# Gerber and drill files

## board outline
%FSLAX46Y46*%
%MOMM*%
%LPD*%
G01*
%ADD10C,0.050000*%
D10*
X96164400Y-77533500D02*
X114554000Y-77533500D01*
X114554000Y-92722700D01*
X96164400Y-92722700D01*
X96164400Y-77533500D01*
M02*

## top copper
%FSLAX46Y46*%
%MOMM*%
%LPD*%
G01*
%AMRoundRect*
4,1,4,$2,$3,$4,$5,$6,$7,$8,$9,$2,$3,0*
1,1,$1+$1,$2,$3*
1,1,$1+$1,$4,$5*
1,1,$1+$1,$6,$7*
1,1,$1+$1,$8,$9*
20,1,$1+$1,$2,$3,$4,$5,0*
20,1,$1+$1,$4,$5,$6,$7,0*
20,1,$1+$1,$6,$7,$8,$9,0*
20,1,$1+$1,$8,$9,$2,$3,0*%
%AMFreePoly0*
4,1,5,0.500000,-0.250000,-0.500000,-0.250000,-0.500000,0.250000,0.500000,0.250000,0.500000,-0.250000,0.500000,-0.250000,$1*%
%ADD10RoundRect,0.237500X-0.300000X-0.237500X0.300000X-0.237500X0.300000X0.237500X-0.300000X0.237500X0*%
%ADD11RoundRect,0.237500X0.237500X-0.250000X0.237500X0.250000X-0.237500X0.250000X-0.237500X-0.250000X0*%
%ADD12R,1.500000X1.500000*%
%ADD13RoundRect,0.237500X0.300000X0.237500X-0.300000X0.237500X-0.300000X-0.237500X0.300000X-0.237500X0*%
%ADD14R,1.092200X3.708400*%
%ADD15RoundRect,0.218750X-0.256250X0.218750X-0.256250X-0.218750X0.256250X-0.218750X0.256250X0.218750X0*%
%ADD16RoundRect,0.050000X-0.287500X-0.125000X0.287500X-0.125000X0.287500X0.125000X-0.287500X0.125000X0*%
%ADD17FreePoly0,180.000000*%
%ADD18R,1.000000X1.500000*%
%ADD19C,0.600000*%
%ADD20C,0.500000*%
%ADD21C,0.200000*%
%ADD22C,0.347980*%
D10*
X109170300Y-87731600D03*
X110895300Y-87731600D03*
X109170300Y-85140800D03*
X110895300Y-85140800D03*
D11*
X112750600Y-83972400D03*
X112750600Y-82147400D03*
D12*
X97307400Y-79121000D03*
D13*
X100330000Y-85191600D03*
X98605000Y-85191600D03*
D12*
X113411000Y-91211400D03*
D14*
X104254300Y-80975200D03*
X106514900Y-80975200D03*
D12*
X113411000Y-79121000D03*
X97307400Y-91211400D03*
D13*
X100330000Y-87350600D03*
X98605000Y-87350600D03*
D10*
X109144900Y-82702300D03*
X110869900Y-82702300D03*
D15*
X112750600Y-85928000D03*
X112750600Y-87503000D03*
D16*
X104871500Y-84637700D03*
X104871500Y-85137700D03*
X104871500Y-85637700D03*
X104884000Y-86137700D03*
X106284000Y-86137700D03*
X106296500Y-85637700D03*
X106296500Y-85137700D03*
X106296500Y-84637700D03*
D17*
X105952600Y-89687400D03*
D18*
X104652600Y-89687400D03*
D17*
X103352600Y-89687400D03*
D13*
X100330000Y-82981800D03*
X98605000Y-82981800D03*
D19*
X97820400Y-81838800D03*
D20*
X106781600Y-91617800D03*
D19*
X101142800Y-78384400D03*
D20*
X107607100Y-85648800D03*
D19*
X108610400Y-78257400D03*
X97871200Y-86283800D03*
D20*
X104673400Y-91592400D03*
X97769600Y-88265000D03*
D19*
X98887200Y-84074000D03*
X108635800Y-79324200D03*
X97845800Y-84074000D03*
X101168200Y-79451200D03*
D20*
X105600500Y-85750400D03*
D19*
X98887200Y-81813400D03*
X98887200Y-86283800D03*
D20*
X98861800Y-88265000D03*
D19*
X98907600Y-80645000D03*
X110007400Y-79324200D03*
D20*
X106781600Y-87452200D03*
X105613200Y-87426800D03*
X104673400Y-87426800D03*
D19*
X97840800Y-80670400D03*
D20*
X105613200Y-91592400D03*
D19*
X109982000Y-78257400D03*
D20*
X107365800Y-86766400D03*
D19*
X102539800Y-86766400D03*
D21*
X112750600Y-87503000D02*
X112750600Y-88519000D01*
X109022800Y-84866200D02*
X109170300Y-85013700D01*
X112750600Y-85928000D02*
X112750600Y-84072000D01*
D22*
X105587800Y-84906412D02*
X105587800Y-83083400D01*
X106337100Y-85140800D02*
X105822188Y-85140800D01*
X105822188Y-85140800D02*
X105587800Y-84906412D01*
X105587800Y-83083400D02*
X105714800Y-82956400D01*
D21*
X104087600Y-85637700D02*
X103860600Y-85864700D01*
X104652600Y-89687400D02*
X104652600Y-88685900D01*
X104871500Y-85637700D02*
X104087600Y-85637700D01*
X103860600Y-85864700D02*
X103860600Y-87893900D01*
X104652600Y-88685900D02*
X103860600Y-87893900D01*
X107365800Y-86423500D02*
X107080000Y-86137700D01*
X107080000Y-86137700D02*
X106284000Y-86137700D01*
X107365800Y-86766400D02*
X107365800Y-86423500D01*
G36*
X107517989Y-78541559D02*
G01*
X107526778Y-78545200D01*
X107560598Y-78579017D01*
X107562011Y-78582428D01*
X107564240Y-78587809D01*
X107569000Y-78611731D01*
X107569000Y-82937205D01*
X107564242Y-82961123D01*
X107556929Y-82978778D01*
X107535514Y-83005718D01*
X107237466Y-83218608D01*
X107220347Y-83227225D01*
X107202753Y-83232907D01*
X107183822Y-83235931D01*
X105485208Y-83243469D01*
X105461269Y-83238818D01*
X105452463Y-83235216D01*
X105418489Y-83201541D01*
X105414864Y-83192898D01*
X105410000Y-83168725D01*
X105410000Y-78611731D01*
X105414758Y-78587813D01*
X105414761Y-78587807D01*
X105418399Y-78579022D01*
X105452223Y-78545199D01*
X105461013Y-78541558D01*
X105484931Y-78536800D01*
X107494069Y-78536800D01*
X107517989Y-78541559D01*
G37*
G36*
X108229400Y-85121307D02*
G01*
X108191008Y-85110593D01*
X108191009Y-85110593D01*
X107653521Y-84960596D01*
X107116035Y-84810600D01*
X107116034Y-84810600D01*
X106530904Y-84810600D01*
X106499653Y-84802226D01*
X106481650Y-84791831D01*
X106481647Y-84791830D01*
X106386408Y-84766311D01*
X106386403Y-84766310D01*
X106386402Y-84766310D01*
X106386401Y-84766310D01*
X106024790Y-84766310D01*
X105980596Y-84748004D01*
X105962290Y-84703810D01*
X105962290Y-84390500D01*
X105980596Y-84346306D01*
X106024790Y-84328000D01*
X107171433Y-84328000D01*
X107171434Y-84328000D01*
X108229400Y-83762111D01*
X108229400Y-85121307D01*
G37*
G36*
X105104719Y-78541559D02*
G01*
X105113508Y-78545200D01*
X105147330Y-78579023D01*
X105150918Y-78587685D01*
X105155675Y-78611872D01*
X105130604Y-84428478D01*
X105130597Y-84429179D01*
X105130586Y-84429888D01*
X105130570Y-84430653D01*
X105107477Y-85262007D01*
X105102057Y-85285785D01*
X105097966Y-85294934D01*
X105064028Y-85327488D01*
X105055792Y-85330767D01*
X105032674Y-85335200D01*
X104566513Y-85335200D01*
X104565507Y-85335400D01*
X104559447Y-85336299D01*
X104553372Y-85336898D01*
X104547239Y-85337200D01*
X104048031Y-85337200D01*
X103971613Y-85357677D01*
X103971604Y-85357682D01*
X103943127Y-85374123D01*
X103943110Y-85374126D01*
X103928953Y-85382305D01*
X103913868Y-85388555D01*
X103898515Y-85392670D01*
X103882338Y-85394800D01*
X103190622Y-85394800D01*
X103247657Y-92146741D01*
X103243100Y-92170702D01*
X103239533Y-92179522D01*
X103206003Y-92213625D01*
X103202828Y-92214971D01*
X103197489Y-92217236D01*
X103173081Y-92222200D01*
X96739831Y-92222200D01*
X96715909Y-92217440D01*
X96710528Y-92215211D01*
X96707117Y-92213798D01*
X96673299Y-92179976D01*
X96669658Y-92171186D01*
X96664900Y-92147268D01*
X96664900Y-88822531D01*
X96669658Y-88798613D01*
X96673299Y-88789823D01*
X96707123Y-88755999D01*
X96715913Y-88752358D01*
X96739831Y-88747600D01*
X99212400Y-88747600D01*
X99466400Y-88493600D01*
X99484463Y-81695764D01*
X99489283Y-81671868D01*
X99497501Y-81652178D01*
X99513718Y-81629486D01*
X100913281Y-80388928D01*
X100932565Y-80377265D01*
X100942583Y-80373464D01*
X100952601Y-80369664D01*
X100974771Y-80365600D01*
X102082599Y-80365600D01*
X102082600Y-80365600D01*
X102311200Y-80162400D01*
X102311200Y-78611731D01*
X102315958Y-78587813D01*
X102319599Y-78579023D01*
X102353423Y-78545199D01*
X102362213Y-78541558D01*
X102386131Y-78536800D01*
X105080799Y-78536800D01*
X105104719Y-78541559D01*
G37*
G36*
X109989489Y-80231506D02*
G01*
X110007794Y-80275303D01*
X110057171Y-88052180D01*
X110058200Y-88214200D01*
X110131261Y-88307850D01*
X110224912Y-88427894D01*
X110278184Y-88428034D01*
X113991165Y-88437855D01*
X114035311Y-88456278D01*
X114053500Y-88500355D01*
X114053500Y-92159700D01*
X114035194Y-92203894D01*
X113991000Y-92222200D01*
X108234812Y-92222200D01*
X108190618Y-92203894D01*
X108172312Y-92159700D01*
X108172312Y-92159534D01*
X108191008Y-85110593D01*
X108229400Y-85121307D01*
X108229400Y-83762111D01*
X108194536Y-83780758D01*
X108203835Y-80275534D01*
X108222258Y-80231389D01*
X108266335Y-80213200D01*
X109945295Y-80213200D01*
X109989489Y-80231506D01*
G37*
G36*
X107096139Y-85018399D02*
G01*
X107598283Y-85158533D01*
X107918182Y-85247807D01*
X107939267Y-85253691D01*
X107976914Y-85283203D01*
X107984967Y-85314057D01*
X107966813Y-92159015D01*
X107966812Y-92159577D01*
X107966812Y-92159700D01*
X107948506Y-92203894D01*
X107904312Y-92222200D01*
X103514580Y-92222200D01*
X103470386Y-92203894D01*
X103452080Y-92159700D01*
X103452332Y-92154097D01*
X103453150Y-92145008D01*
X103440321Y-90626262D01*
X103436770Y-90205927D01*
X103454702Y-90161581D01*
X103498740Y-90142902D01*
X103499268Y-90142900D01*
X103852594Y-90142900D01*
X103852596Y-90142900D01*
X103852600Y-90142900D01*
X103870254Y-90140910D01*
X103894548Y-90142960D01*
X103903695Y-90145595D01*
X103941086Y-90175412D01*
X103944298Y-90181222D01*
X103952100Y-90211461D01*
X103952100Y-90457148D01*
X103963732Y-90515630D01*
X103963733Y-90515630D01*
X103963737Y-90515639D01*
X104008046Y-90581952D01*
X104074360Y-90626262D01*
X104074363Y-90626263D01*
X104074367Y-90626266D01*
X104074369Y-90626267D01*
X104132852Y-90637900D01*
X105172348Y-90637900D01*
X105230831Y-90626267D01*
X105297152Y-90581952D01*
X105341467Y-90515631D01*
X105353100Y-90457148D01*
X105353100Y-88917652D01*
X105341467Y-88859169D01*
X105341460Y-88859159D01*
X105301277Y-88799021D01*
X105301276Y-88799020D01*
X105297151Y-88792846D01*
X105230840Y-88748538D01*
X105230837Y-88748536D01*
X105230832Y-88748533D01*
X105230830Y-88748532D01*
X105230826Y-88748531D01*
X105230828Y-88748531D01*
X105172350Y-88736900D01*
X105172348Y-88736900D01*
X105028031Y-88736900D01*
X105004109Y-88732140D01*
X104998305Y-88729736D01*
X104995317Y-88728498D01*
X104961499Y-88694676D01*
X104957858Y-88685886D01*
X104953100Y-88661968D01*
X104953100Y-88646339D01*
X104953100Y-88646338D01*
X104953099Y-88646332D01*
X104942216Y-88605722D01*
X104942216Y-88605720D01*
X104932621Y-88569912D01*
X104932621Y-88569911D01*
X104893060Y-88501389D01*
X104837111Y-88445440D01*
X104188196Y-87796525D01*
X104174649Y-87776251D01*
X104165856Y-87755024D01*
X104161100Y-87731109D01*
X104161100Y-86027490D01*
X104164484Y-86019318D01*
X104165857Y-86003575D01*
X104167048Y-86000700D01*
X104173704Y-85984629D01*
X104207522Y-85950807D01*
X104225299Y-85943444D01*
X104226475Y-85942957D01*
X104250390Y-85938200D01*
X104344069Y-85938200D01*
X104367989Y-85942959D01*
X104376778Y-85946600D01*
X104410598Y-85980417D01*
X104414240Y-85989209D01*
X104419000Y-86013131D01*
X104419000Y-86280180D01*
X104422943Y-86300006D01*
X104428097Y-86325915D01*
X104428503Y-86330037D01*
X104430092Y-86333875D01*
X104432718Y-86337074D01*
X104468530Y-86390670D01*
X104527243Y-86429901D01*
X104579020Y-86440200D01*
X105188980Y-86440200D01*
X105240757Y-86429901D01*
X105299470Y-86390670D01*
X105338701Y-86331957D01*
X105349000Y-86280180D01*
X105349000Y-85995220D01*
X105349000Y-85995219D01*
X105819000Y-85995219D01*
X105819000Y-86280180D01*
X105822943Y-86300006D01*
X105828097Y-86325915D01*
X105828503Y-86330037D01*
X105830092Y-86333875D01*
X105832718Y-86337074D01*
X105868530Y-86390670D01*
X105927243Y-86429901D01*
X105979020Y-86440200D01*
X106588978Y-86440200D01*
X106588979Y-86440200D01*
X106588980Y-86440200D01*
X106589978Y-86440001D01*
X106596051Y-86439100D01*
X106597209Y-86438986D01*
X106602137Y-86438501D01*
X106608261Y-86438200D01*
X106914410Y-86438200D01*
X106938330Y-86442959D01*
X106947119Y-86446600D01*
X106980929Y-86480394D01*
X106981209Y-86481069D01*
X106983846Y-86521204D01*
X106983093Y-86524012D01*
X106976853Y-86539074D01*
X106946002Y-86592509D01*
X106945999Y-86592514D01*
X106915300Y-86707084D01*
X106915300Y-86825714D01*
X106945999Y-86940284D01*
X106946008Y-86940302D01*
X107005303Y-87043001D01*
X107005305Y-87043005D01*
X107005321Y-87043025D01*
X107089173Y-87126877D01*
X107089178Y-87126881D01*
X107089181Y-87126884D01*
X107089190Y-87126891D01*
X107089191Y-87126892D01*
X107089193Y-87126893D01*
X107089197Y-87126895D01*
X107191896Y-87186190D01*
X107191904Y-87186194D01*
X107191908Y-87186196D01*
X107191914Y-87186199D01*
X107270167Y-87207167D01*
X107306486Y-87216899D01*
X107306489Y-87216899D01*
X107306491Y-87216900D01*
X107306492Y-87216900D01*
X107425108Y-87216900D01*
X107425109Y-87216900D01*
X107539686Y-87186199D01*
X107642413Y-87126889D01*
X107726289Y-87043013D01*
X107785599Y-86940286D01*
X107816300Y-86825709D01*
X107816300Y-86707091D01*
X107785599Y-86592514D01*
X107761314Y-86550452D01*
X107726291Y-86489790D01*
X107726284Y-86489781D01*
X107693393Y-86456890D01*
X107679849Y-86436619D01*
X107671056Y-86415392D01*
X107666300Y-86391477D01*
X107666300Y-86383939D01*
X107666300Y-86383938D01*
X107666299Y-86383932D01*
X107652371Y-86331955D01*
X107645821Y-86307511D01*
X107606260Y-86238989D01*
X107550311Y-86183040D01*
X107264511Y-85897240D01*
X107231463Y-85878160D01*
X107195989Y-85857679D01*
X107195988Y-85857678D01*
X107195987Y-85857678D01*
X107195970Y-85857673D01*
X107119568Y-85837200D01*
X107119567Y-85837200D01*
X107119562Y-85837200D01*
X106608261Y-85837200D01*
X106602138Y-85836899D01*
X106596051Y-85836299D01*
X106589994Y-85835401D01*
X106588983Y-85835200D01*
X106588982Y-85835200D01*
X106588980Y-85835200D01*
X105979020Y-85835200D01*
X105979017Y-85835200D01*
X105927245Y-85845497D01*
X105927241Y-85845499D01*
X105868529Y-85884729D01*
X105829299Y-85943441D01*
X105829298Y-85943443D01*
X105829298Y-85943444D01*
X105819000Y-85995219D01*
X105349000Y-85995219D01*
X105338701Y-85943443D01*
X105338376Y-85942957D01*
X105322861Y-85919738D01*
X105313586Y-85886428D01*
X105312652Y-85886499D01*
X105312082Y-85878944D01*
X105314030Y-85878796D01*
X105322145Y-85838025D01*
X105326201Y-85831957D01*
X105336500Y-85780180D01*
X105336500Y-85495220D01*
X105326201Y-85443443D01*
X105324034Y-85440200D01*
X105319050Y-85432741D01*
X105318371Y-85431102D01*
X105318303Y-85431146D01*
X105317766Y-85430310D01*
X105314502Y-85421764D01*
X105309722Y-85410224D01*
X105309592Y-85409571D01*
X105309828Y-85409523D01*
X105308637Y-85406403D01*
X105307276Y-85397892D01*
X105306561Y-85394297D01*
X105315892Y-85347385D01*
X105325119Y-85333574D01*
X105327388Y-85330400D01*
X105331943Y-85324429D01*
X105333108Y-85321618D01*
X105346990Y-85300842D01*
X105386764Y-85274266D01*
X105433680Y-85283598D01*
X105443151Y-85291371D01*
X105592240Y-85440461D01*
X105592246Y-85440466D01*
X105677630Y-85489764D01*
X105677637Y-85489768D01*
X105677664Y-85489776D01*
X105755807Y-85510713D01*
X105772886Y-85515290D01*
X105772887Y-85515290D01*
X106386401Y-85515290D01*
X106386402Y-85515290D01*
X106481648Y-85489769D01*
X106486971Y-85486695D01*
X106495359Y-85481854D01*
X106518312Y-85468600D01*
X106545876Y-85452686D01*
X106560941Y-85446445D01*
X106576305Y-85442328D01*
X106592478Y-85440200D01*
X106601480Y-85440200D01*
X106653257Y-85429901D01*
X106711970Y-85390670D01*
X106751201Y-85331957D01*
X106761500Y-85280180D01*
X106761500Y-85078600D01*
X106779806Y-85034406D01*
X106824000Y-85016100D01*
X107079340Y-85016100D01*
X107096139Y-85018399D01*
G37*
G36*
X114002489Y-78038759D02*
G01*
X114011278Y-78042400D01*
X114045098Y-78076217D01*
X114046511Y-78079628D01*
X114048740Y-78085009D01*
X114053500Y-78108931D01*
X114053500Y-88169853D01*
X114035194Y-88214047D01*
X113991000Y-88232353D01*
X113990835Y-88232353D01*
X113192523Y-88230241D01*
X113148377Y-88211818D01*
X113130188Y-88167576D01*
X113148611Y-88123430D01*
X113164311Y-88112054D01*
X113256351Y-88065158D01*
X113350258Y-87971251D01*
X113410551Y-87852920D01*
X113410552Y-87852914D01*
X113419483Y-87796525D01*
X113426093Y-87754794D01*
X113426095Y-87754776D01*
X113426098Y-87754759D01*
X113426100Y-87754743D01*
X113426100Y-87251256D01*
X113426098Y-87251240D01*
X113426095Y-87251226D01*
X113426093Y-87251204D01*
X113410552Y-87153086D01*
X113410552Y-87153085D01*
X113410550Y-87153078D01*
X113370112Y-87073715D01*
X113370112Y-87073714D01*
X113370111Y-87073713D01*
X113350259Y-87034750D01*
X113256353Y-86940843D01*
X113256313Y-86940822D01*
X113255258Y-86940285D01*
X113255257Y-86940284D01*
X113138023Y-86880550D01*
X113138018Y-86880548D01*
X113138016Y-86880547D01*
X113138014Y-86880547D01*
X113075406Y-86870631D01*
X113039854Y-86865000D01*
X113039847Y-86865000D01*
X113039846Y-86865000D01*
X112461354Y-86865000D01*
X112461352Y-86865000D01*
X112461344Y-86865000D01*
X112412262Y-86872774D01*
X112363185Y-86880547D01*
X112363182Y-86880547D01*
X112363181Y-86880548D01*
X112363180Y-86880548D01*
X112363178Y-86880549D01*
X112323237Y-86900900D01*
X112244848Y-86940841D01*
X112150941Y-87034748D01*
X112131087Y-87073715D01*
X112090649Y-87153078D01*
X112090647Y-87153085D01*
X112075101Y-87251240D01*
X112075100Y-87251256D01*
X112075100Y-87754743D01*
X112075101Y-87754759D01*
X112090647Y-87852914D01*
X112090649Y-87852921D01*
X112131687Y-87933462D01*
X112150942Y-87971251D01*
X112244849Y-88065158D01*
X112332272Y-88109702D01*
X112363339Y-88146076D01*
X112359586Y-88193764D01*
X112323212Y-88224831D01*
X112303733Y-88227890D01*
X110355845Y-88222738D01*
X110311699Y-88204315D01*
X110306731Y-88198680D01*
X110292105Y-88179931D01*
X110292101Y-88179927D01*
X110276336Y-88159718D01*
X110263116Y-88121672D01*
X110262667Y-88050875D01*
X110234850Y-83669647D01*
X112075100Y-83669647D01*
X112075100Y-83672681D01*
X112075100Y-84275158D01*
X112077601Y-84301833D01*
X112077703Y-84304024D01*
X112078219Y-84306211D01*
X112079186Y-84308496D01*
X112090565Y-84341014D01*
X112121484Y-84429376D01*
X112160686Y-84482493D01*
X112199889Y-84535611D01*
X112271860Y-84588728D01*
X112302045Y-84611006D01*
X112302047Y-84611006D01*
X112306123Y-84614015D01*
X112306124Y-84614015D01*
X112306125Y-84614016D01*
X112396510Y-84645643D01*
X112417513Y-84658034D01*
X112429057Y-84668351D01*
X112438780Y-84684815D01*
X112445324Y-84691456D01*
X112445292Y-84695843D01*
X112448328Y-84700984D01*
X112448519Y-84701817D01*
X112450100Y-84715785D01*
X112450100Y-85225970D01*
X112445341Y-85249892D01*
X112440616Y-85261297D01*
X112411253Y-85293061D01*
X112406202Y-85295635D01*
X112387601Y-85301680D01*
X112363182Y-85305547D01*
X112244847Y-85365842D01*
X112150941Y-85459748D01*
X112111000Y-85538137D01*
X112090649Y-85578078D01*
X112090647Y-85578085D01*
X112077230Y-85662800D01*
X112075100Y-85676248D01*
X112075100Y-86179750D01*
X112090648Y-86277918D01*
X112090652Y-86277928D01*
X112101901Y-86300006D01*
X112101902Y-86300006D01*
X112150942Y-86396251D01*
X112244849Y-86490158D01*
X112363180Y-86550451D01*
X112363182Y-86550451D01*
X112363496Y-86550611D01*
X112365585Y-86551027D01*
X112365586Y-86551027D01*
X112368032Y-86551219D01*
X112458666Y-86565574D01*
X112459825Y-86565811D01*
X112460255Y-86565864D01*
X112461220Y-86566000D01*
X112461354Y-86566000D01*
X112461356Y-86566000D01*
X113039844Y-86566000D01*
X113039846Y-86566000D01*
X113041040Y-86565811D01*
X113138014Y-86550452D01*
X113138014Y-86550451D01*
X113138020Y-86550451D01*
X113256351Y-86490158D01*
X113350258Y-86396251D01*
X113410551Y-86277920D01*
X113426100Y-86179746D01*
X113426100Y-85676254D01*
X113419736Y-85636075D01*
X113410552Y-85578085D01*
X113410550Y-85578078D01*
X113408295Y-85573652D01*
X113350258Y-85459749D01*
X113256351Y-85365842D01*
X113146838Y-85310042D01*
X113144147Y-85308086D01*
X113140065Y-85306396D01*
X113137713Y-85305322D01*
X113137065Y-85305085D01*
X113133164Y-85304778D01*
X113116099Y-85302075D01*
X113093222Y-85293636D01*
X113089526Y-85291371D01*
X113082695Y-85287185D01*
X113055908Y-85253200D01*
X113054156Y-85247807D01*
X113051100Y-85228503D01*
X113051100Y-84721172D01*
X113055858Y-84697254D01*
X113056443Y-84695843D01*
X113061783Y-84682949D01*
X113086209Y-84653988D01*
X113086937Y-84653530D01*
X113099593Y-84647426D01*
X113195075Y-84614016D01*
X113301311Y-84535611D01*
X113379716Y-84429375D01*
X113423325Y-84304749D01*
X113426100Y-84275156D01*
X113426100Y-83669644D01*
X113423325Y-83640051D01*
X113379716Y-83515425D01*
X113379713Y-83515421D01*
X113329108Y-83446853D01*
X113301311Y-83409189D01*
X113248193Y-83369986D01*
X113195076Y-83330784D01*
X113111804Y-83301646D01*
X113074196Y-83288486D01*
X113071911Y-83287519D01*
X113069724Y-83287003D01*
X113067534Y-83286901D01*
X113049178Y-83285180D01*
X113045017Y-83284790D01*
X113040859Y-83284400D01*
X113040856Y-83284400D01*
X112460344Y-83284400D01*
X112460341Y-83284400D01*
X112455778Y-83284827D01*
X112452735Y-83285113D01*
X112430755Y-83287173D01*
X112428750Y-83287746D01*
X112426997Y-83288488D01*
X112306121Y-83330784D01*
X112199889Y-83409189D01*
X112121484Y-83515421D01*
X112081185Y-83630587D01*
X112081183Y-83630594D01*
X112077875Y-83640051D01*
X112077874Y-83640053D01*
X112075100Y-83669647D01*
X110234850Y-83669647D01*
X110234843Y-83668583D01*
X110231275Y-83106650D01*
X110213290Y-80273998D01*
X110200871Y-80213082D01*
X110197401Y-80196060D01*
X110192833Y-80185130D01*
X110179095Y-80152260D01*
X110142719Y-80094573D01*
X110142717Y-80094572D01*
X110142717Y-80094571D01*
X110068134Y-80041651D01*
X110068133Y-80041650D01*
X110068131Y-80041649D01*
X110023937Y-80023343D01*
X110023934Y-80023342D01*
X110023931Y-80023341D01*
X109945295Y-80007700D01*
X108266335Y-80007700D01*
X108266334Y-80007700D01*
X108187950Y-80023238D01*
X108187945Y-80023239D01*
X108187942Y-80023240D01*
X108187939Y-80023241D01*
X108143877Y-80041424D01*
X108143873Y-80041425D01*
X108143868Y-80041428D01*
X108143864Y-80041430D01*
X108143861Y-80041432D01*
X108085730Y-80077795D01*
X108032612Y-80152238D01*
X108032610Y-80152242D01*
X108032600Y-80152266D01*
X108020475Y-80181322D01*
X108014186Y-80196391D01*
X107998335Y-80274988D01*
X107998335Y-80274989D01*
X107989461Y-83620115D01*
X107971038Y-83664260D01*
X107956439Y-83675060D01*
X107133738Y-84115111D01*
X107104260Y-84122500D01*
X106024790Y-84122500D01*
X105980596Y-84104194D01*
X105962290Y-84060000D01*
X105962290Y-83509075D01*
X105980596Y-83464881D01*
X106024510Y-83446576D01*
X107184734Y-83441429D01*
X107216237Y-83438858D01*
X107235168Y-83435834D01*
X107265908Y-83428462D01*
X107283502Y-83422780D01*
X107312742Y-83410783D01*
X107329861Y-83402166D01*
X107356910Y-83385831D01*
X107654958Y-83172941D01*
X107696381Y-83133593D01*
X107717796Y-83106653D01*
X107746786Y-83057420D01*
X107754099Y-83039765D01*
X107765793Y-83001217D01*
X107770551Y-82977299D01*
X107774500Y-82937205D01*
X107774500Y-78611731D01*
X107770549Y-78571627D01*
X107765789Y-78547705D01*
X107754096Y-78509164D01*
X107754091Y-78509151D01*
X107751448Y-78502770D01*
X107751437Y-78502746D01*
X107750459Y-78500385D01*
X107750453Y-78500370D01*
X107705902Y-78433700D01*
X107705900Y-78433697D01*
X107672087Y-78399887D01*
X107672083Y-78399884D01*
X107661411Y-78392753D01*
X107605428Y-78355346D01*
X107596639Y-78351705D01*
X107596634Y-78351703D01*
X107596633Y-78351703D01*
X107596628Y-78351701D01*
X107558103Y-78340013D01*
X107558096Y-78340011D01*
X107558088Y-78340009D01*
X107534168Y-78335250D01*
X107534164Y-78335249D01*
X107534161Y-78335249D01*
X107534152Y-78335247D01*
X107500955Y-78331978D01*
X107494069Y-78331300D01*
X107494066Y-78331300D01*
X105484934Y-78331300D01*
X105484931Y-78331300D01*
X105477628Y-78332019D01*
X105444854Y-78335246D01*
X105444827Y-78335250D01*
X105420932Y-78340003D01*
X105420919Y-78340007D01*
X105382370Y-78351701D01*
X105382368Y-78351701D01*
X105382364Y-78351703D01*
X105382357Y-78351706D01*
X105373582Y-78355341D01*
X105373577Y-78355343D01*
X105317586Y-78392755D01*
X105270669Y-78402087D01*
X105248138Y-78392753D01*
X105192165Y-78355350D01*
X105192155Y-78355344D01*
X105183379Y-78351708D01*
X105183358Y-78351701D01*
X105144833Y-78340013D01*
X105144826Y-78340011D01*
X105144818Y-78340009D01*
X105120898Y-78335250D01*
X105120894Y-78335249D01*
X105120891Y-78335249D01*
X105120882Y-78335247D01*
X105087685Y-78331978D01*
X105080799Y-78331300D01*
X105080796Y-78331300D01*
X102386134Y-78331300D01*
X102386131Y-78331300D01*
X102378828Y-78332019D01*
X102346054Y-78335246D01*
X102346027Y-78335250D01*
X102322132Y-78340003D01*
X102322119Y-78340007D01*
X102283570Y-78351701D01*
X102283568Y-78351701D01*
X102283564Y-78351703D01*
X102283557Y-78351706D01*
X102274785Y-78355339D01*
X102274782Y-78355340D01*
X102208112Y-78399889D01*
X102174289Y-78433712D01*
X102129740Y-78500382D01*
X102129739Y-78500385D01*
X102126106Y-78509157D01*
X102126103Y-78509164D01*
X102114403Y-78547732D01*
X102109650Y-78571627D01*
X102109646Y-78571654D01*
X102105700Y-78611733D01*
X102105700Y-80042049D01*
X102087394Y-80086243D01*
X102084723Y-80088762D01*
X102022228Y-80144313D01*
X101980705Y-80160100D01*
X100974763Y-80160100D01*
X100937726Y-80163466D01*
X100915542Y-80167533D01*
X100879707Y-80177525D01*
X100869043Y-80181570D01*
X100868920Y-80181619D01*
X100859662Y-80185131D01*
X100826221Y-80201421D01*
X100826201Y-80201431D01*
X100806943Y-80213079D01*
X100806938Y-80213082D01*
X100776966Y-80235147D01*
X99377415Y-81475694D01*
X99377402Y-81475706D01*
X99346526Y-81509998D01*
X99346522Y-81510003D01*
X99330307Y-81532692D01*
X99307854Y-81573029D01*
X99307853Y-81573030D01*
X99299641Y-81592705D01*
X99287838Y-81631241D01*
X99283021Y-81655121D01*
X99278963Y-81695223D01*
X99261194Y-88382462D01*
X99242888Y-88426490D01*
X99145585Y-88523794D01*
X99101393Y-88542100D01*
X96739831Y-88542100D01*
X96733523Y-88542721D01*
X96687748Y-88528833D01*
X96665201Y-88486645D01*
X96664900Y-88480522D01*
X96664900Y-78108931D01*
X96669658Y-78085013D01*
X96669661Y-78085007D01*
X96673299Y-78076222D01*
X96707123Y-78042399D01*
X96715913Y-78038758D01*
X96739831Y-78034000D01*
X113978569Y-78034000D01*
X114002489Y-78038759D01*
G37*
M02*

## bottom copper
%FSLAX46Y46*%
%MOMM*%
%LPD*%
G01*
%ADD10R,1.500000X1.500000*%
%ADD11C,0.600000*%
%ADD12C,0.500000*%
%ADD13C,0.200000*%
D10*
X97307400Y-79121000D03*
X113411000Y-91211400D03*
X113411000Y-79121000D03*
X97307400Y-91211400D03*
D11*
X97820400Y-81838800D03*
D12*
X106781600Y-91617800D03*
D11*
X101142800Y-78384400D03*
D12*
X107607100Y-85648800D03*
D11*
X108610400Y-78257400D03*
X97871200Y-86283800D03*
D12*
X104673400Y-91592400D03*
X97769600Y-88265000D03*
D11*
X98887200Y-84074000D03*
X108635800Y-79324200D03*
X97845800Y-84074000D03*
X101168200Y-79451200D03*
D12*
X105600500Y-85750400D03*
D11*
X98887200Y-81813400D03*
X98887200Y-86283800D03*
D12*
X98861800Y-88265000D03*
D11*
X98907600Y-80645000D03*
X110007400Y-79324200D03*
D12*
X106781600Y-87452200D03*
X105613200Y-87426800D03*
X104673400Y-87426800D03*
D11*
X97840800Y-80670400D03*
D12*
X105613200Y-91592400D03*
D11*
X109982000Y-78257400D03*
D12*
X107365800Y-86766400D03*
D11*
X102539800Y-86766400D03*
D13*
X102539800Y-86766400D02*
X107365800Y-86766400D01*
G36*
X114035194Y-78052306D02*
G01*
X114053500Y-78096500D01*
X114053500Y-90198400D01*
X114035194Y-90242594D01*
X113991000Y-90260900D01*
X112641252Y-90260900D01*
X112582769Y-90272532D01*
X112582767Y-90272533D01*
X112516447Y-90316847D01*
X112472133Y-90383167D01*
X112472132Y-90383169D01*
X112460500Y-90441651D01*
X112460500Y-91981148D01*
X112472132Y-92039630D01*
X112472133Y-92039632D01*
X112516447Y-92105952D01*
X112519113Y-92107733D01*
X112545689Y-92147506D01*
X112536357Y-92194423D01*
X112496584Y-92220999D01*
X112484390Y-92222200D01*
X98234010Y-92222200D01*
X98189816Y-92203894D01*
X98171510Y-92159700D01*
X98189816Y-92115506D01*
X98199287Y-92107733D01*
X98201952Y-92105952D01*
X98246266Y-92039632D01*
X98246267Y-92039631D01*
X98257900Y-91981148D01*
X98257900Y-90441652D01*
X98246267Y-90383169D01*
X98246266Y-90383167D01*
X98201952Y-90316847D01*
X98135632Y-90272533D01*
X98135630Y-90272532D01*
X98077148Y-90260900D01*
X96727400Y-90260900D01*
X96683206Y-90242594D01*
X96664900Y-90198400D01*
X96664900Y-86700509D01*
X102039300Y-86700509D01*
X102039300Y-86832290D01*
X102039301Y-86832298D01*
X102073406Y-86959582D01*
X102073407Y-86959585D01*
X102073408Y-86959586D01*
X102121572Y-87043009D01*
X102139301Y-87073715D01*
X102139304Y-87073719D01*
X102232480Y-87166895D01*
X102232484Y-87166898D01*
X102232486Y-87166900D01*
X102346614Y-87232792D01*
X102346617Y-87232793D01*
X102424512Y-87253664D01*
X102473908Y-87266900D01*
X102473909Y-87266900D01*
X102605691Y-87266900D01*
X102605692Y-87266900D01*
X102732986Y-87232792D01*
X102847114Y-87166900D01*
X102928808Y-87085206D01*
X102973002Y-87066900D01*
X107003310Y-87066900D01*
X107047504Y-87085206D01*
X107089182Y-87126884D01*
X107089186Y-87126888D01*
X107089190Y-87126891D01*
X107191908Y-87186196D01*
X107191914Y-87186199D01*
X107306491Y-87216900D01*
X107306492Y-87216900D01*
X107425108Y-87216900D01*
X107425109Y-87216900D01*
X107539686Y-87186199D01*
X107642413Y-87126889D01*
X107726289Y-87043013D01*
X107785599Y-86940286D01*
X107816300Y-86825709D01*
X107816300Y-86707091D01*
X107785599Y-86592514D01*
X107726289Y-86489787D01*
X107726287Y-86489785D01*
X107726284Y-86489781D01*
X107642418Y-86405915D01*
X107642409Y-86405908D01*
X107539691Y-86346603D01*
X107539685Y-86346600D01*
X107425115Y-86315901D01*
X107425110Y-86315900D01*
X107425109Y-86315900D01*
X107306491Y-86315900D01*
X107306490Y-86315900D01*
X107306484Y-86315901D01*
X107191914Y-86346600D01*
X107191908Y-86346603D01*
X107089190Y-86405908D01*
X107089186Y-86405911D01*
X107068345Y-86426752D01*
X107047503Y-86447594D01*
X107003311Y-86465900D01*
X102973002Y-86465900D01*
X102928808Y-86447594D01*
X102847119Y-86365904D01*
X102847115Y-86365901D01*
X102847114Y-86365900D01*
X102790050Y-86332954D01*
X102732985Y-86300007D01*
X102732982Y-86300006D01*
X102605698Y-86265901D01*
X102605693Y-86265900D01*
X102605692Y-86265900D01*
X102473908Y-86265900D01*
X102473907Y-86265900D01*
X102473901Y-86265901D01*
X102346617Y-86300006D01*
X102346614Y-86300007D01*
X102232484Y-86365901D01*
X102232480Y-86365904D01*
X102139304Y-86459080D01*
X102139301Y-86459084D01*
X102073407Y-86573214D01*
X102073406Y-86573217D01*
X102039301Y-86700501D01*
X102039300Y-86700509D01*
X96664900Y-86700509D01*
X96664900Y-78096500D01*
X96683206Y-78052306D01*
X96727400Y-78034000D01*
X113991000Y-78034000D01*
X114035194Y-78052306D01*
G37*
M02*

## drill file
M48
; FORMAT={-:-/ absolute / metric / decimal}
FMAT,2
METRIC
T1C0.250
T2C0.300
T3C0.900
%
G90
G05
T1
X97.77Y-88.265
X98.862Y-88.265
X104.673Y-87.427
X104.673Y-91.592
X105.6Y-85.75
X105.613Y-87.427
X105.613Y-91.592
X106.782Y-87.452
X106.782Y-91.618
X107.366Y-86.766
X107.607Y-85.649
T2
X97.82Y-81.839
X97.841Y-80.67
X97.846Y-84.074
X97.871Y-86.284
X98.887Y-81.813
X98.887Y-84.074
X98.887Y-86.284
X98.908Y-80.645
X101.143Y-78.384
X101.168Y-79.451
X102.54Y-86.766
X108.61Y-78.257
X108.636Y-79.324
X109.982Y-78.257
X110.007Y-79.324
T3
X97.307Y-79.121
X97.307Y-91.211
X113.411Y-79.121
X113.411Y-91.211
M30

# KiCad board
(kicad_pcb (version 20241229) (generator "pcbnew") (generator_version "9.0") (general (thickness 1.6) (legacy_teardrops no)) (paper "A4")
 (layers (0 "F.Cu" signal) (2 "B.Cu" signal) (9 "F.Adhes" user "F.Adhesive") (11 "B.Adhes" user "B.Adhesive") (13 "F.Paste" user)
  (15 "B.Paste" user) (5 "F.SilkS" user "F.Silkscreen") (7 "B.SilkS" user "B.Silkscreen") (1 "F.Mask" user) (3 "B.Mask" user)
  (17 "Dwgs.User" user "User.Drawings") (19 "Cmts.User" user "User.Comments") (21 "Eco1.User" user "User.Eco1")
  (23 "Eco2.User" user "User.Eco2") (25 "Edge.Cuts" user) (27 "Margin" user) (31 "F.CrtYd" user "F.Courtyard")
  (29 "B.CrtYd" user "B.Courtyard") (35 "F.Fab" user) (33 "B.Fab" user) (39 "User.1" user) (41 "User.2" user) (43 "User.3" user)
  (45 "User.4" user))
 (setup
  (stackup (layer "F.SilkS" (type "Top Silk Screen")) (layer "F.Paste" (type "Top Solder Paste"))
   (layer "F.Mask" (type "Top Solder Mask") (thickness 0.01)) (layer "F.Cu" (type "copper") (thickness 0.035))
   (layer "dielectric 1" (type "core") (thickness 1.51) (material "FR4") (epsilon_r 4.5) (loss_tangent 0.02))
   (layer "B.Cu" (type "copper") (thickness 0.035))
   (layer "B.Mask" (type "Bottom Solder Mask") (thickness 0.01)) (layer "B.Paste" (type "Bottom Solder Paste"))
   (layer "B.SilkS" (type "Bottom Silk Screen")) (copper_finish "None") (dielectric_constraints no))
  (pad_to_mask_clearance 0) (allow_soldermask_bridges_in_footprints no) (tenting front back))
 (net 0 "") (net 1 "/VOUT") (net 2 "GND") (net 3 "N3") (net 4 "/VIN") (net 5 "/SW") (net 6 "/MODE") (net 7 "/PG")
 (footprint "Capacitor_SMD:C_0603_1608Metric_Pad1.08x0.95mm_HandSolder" (layer "F.Cu") (at 110.0328 87.7316)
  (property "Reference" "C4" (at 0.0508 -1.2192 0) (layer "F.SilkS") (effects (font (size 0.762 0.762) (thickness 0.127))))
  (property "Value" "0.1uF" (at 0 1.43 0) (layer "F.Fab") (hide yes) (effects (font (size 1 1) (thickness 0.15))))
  (pad "1" smd roundrect (at -0.8625 0) (size 1.075 0.95) (layers "F.Cu" "F.Mask" "F.Paste") (roundrect_rratio 0.25) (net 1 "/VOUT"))
  (pad "2" smd roundrect (at 0.8625 0) (size 1.075 0.95) (layers "F.Cu" "F.Mask" "F.Paste") (roundrect_rratio 0.25) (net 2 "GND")))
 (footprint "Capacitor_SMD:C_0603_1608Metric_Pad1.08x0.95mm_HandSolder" (layer "F.Cu") (at 110.0328 85.1408)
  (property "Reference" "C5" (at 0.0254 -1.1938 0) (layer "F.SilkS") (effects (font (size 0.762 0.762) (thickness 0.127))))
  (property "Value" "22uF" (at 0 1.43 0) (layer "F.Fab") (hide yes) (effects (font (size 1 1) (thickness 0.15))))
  (pad "1" smd roundrect (at -0.8625 0) (size 1.075 0.95) (layers "F.Cu" "F.Mask" "F.Paste") (roundrect_rratio 0.25) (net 1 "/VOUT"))
  (pad "2" smd roundrect (at 0.8625 0) (size 1.075 0.95) (layers "F.Cu" "F.Mask" "F.Paste") (roundrect_rratio 0.25) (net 2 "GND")))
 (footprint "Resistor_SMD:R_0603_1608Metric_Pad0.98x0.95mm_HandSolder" (layer "F.Cu") (at 112.7506 83.0599 90)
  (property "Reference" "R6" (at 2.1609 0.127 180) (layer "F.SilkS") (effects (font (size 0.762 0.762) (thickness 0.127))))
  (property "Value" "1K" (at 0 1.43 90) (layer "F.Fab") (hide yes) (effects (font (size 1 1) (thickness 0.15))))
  (pad "1" smd roundrect (at -0.9125 0 90) (size 0.975 0.95) (layers "F.Cu" "F.Mask" "F.Paste") (roundrect_rratio 0.25) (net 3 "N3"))
  (pad "2" smd roundrect (at 0.9125 0 90) (size 0.975 0.95) (layers "F.Cu" "F.Mask" "F.Paste") (roundrect_rratio 0.25) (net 2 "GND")))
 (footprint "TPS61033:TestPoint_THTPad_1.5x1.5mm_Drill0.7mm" (layer "F.Cu") (at 97.3074 79.121)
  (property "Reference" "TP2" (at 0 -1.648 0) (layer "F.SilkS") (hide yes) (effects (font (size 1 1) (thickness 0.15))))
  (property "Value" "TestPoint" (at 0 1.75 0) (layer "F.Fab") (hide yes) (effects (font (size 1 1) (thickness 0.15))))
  (pad "1" thru_hole rect (at 0 0) (size 1.5 1.5) (drill 0.9) (layers "*.Cu" "*.Mask") (remove_unused_layers no) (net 2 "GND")))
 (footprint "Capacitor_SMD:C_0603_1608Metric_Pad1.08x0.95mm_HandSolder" (layer "F.Cu") (at 99.4675 85.1916 180)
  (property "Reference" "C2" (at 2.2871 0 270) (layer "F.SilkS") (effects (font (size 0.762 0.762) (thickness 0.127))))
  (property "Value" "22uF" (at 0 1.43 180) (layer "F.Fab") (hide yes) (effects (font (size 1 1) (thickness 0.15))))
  (pad "1" smd roundrect (at -0.8625 0 180) (size 1.075 0.95) (layers "F.Cu" "F.Mask" "F.Paste") (roundrect_rratio 0.25) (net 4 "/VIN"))
  (pad "2" smd roundrect (at 0.8625 0 180) (size 1.075 0.95) (layers "F.Cu" "F.Mask" "F.Paste") (roundrect_rratio 0.25) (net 2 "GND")))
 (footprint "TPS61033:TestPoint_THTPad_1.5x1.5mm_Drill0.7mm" (layer "F.Cu") (at 113.411 91.2114)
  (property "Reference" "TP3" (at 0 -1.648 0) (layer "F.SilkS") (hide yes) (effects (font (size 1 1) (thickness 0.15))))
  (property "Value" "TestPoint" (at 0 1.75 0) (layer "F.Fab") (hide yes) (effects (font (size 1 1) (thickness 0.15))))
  (pad "1" thru_hole rect (at 0 0) (size 1.5 1.5) (drill 0.9) (layers "*.Cu" "*.Mask") (remove_unused_layers no) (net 1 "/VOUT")))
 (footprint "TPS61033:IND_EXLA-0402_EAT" (layer "F.Cu") (at 105.3846 80.9752)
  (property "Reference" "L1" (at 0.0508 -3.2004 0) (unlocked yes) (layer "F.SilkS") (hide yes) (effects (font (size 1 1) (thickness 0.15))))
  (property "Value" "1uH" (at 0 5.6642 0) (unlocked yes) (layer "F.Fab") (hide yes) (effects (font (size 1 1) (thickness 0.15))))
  (pad "1" smd rect (at -1.1303 0) (size 1.0922 3.7084) (layers "F.Cu" "F.Mask" "F.Paste") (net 4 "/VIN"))
  (pad "2" smd rect (at 1.1303 0) (size 1.0922 3.7084) (layers "F.Cu" "F.Mask" "F.Paste") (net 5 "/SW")))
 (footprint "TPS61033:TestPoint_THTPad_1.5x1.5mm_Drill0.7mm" (layer "F.Cu") (at 113.411 79.121)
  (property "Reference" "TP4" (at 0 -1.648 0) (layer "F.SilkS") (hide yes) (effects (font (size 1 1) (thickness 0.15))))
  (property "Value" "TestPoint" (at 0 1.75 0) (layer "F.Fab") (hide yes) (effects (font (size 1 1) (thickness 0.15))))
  (pad "1" thru_hole rect (at 0 0) (size 1.5 1.5) (drill 0.9) (layers "*.Cu" "*.Mask") (remove_unused_layers no) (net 2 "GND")))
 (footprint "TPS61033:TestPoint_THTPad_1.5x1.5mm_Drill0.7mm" (layer "F.Cu") (at 97.3074 91.2114)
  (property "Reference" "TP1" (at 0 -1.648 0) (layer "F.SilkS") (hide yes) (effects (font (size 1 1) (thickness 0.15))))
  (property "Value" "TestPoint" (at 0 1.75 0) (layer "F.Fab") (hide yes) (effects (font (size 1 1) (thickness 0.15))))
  (pad "1" thru_hole rect (at 0 0) (size 1.5 1.5) (drill 0.9) (layers "*.Cu" "*.Mask") (remove_unused_layers no) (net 4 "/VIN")))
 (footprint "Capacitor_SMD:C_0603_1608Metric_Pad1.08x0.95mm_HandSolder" (layer "F.Cu") (at 99.4675 87.3506 180)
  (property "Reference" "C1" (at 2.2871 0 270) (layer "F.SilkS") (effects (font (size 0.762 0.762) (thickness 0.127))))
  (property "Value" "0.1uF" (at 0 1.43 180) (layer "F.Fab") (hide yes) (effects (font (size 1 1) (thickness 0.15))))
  (pad "1" smd roundrect (at -0.8625 0 180) (size 1.075 0.95) (layers "F.Cu" "F.Mask" "F.Paste") (roundrect_rratio 0.25) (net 4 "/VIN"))
  (pad "2" smd roundrect (at 0.8625 0 180) (size 1.075 0.95) (layers "F.Cu" "F.Mask" "F.Paste") (roundrect_rratio 0.25) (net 2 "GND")))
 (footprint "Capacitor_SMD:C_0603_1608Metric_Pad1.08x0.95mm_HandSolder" (layer "F.Cu") (at 110.0074 82.7023)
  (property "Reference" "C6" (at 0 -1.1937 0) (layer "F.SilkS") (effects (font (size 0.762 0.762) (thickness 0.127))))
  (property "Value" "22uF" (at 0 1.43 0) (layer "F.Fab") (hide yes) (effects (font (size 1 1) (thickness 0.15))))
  (pad "1" smd roundrect (at -0.8625 0) (size 1.075 0.95) (layers "F.Cu" "F.Mask" "F.Paste") (roundrect_rratio 0.25) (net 1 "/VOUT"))
  (pad "2" smd roundrect (at 0.8625 0) (size 1.075 0.95) (layers "F.Cu" "F.Mask" "F.Paste") (roundrect_rratio 0.25) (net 2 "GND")))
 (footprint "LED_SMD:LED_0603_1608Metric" (layer "F.Cu") (at 112.7506 86.7155 -90)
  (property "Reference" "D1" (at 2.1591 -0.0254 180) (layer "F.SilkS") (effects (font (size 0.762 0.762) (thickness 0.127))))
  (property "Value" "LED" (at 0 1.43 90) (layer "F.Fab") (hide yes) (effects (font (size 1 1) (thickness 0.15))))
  (pad "1" smd roundrect (at -0.7875 0 270) (size 0.875 0.95) (layers "F.Cu" "F.Mask" "F.Paste") (roundrect_rratio 0.25) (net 3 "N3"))
  (pad "2" smd roundrect (at 0.7875 0 270) (size 0.875 0.95) (layers "F.Cu" "F.Mask" "F.Paste") (roundrect_rratio 0.25) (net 1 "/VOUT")))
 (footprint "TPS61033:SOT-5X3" (layer "F.Cu") (at 105.584 85.1377)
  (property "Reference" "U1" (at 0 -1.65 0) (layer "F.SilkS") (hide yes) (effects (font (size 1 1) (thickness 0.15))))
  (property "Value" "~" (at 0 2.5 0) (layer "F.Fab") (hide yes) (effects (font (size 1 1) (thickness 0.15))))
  (pad "1" smd roundrect (at -0.7125 -0.5) (size 0.675 0.35) (layers "F.Cu" "F.Mask" "F.Paste") (roundrect_rratio 0.1428571429)
   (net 4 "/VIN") (clearance 0.127))
  (pad "2" smd roundrect (at -0.7125 0) (size 0.675 0.35) (layers "F.Cu" "F.Mask" "F.Paste") (roundrect_rratio 0.1428571429) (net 4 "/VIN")
   (clearance 0.127))
  (pad "3" smd roundrect (at -0.7125 0.5) (size 0.675 0.35) (layers "F.Cu" "F.Mask" "F.Paste") (roundrect_rratio 0.1428571429)
   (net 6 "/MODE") (clearance 0.127))
  (pad "4" smd roundrect (at -0.7 1) (size 0.675 0.35) (layers "F.Cu" "F.Mask" "F.Paste") (roundrect_rratio 0.1428571429) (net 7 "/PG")
   (clearance 0.127))
  (pad "5" smd roundrect (at 0.7 1) (size 0.675 0.35) (layers "F.Cu" "F.Mask" "F.Paste") (roundrect_rratio 0.1428571429) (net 4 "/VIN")
   (clearance 0.127))
  (pad "6" smd roundrect (at 0.7125 0.5) (size 0.675 0.35) (layers "F.Cu" "F.Mask" "F.Paste") (roundrect_rratio 0.1428571429) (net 2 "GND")
   (clearance 0.127))
  (pad "7" smd roundrect (at 0.7125 0) (size 0.675 0.35) (layers "F.Cu" "F.Mask" "F.Paste") (roundrect_rratio 0.1428571429) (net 5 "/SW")
   (clearance 0.127))
  (pad "8" smd roundrect (at 0.7125 -0.5) (size 0.675 0.35) (layers "F.Cu" "F.Mask" "F.Paste") (roundrect_rratio 0.1428571429)
   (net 1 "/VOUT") (clearance 0.127)))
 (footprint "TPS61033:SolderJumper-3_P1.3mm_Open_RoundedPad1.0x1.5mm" (layer "F.Cu") (at 104.6526 89.6874 180)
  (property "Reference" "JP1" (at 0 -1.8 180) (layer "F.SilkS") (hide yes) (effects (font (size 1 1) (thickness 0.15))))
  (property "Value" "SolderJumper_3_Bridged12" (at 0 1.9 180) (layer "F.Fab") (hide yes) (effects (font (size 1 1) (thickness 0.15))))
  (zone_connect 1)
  (pad "1" smd custom (at -1.3 0 180) (size 1 0.5) (layers "F.Cu" "F.Mask") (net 2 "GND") (zone_connect 2) (thermal_bridge_angle 45)
   (options (clearance outline) (anchor rect)) (primitives))
  (pad "2" smd rect (at 0 0 180) (size 1 1.5) (layers "F.Cu" "F.Mask") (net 6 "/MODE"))
  (pad "3" smd custom (at 1.3 0 180) (size 1 0.5) (layers "F.Cu" "F.Mask") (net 4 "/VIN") (zone_connect 2) (thermal_bridge_angle 45)
   (options (clearance outline) (anchor rect)) (primitives)))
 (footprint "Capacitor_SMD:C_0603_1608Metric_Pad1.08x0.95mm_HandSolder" (layer "F.Cu") (at 99.4675 82.9818 180)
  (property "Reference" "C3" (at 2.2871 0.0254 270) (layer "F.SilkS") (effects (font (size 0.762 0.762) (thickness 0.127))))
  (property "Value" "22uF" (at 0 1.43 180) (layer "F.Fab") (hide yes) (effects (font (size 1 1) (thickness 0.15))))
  (pad "1" smd roundrect (at -0.8625 0 180) (size 1.075 0.95) (layers "F.Cu" "F.Mask" "F.Paste") (roundrect_rratio 0.25) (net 4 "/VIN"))
  (pad "2" smd roundrect (at 0.8625 0 180) (size 1.075 0.95) (layers "F.Cu" "F.Mask" "F.Paste") (roundrect_rratio 0.25) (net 2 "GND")))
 (gr_rect (start 96.1644 77.5335) (end 114.554 92.7227) (stroke (width 0.05) (type default)) (fill no) (layer "Edge.Cuts"))
 (via (at 97.8204 81.8388) (size 0.6) (drill 0.3) (layers "F.Cu" "B.Cu") (free yes) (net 2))
 (via (at 106.7816 91.6178) (size 0.5) (drill 0.25) (layers "F.Cu" "B.Cu") (free yes) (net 2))
 (via (at 101.1428 78.3844) (size 0.6) (drill 0.3) (layers "F.Cu" "B.Cu") (free yes) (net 2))
 (via (at 107.6071 85.6488) (size 0.5) (drill 0.25) (layers "F.Cu" "B.Cu") (free yes) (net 2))
 (via (at 108.6104 78.2574) (size 0.6) (drill 0.3) (layers "F.Cu" "B.Cu") (free yes) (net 2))
 (via (at 97.8712 86.2838) (size 0.6) (drill 0.3) (layers "F.Cu" "B.Cu") (free yes) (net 2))
 (via (at 104.6734 91.5924) (size 0.5) (drill 0.25) (layers "F.Cu" "B.Cu") (free yes) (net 2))
 (via (at 97.7696 88.265) (size 0.5) (drill 0.25) (layers "F.Cu" "B.Cu") (free yes) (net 2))
 (via (at 98.8872 84.074) (size 0.6) (drill 0.3) (layers "F.Cu" "B.Cu") (free yes) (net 2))
 (via (at 108.6358 79.3242) (size 0.6) (drill 0.3) (layers "F.Cu" "B.Cu") (free yes) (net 2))
 (via (at 97.8458 84.074) (size 0.6) (drill 0.3) (layers "F.Cu" "B.Cu") (free yes) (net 2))
 (via (at 101.1682 79.4512) (size 0.6) (drill 0.3) (layers "F.Cu" "B.Cu") (free yes) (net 2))
 (via (at 105.6005 85.7504) (size 0.5) (drill 0.25) (layers "F.Cu" "B.Cu") (free yes) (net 2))
 (via (at 98.8872 81.8134) (size 0.6) (drill 0.3) (layers "F.Cu" "B.Cu") (free yes) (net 2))
 (via (at 98.8872 86.2838) (size 0.6) (drill 0.3) (layers "F.Cu" "B.Cu") (free yes) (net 2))
 (via (at 98.8618 88.265) (size 0.5) (drill 0.25) (layers "F.Cu" "B.Cu") (free yes) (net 2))
 (via (at 98.9076 80.645) (size 0.6) (drill 0.3) (layers "F.Cu" "B.Cu") (free yes) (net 2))
 (via (at 110.0074 79.3242) (size 0.6) (drill 0.3) (layers "F.Cu" "B.Cu") (free yes) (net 2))
 (via (at 106.7816 87.4522) (size 0.5) (drill 0.25) (layers "F.Cu" "B.Cu") (free yes) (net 2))
 (via (at 105.6132 87.4268) (size 0.5) (drill 0.25) (layers "F.Cu" "B.Cu") (free yes) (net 2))
 (via (at 104.6734 87.4268) (size 0.5) (drill 0.25) (layers "F.Cu" "B.Cu") (free yes) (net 2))
 (via (at 97.8408 80.6704) (size 0.6) (drill 0.3) (layers "F.Cu" "B.Cu") (free yes) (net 2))
 (via (at 105.6132 91.5924) (size 0.5) (drill 0.25) (layers "F.Cu" "B.Cu") (free yes) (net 2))
 (via (at 109.982 78.2574) (size 0.6) (drill 0.3) (layers "F.Cu" "B.Cu") (free yes) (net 2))
 (segment (start 112.7506 87.503) (end 112.7506 88.519) (width 0.2) (layer "F.Cu") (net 1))
 (segment (start 109.0228 84.8662) (end 109.1703 85.0137) (width 0.2) (layer "F.Cu") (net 1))
 (segment (start 112.7506 85.928) (end 112.7506 84.072) (width 0.2) (layer "F.Cu") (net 3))
 (segment (start 105.5878 84.906412) (end 105.5878 83.0834) (width 0.34798) (layer "F.Cu") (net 5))
 (segment (start 106.3371 85.1408) (end 105.822188 85.1408) (width 0.34798) (layer "F.Cu") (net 5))
 (segment (start 105.822188 85.1408) (end 105.5878 84.906412) (width 0.34798) (layer "F.Cu") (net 5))
 (segment (start 105.5878 83.0834) (end 105.7148 82.9564) (width 0.34798) (layer "F.Cu") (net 5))
 (segment (start 104.0876 85.6377) (end 103.8606 85.8647) (width 0.2) (layer "F.Cu") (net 6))
 (segment (start 104.6526 89.6874) (end 104.6526 88.6859) (width 0.2) (layer "F.Cu") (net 6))
 (segment (start 104.8715 85.6377) (end 104.0876 85.6377) (width 0.2) (layer "F.Cu") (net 6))
 (segment (start 103.8606 85.8647) (end 103.8606 87.8939) (width 0.2) (layer "F.Cu") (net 6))
 (segment (start 104.6526 88.6859) (end 103.8606 87.8939) (width 0.2) (layer "F.Cu") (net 6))
 (segment (start 107.3658 86.4235) (end 107.08 86.1377) (width 0.2) (layer "F.Cu") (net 4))
 (segment (start 107.08 86.1377) (end 106.284 86.1377) (width 0.2) (layer "F.Cu") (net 4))
 (segment (start 107.3658 86.7664) (end 107.3658 86.4235) (width 0.2) (layer "F.Cu") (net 4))
 (via (at 107.3658 86.7664) (size 0.5) (drill 0.25) (layers "F.Cu" "B.Cu") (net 4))
 (via (at 102.5398 86.7664) (size 0.6) (drill 0.3) (layers "F.Cu" "B.Cu") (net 4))
 (segment (start 102.5398 86.7664) (end 107.3658 86.7664) (width 0.2) (layer "B.Cu") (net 4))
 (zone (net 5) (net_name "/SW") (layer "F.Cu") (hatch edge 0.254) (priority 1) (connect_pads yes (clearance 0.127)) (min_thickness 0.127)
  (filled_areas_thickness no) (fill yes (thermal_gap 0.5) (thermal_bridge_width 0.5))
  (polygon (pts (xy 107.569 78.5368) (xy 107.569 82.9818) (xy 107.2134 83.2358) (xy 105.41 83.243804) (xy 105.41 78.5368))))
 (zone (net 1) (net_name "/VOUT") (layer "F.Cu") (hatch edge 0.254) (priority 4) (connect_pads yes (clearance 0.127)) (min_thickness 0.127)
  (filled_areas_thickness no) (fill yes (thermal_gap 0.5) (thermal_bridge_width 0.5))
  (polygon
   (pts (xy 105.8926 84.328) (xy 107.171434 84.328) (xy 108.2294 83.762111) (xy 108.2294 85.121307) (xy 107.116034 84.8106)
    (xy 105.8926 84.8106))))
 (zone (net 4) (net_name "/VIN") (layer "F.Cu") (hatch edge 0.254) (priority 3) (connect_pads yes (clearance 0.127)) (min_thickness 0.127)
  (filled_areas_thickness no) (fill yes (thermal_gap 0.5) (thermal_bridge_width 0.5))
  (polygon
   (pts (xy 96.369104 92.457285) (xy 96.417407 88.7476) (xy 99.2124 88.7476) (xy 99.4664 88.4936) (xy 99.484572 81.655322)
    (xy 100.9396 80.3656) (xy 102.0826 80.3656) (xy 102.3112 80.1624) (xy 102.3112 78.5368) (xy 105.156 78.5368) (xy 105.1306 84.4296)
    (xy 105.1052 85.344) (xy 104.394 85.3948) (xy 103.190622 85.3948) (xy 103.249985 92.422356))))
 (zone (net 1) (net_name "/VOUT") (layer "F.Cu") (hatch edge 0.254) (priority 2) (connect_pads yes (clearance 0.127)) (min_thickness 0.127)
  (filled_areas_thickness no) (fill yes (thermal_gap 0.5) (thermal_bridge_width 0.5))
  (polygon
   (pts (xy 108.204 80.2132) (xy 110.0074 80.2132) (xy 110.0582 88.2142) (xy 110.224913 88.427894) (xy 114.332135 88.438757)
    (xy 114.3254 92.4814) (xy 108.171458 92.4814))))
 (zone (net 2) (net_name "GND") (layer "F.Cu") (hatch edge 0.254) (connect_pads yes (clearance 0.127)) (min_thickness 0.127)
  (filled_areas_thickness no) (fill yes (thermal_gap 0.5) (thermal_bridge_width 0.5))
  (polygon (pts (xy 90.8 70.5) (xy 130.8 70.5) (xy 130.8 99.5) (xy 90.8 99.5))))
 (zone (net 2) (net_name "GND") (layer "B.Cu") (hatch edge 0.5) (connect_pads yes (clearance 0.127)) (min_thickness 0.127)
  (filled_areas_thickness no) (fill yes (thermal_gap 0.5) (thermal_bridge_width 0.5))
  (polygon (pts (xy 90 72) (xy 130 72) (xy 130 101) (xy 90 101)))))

